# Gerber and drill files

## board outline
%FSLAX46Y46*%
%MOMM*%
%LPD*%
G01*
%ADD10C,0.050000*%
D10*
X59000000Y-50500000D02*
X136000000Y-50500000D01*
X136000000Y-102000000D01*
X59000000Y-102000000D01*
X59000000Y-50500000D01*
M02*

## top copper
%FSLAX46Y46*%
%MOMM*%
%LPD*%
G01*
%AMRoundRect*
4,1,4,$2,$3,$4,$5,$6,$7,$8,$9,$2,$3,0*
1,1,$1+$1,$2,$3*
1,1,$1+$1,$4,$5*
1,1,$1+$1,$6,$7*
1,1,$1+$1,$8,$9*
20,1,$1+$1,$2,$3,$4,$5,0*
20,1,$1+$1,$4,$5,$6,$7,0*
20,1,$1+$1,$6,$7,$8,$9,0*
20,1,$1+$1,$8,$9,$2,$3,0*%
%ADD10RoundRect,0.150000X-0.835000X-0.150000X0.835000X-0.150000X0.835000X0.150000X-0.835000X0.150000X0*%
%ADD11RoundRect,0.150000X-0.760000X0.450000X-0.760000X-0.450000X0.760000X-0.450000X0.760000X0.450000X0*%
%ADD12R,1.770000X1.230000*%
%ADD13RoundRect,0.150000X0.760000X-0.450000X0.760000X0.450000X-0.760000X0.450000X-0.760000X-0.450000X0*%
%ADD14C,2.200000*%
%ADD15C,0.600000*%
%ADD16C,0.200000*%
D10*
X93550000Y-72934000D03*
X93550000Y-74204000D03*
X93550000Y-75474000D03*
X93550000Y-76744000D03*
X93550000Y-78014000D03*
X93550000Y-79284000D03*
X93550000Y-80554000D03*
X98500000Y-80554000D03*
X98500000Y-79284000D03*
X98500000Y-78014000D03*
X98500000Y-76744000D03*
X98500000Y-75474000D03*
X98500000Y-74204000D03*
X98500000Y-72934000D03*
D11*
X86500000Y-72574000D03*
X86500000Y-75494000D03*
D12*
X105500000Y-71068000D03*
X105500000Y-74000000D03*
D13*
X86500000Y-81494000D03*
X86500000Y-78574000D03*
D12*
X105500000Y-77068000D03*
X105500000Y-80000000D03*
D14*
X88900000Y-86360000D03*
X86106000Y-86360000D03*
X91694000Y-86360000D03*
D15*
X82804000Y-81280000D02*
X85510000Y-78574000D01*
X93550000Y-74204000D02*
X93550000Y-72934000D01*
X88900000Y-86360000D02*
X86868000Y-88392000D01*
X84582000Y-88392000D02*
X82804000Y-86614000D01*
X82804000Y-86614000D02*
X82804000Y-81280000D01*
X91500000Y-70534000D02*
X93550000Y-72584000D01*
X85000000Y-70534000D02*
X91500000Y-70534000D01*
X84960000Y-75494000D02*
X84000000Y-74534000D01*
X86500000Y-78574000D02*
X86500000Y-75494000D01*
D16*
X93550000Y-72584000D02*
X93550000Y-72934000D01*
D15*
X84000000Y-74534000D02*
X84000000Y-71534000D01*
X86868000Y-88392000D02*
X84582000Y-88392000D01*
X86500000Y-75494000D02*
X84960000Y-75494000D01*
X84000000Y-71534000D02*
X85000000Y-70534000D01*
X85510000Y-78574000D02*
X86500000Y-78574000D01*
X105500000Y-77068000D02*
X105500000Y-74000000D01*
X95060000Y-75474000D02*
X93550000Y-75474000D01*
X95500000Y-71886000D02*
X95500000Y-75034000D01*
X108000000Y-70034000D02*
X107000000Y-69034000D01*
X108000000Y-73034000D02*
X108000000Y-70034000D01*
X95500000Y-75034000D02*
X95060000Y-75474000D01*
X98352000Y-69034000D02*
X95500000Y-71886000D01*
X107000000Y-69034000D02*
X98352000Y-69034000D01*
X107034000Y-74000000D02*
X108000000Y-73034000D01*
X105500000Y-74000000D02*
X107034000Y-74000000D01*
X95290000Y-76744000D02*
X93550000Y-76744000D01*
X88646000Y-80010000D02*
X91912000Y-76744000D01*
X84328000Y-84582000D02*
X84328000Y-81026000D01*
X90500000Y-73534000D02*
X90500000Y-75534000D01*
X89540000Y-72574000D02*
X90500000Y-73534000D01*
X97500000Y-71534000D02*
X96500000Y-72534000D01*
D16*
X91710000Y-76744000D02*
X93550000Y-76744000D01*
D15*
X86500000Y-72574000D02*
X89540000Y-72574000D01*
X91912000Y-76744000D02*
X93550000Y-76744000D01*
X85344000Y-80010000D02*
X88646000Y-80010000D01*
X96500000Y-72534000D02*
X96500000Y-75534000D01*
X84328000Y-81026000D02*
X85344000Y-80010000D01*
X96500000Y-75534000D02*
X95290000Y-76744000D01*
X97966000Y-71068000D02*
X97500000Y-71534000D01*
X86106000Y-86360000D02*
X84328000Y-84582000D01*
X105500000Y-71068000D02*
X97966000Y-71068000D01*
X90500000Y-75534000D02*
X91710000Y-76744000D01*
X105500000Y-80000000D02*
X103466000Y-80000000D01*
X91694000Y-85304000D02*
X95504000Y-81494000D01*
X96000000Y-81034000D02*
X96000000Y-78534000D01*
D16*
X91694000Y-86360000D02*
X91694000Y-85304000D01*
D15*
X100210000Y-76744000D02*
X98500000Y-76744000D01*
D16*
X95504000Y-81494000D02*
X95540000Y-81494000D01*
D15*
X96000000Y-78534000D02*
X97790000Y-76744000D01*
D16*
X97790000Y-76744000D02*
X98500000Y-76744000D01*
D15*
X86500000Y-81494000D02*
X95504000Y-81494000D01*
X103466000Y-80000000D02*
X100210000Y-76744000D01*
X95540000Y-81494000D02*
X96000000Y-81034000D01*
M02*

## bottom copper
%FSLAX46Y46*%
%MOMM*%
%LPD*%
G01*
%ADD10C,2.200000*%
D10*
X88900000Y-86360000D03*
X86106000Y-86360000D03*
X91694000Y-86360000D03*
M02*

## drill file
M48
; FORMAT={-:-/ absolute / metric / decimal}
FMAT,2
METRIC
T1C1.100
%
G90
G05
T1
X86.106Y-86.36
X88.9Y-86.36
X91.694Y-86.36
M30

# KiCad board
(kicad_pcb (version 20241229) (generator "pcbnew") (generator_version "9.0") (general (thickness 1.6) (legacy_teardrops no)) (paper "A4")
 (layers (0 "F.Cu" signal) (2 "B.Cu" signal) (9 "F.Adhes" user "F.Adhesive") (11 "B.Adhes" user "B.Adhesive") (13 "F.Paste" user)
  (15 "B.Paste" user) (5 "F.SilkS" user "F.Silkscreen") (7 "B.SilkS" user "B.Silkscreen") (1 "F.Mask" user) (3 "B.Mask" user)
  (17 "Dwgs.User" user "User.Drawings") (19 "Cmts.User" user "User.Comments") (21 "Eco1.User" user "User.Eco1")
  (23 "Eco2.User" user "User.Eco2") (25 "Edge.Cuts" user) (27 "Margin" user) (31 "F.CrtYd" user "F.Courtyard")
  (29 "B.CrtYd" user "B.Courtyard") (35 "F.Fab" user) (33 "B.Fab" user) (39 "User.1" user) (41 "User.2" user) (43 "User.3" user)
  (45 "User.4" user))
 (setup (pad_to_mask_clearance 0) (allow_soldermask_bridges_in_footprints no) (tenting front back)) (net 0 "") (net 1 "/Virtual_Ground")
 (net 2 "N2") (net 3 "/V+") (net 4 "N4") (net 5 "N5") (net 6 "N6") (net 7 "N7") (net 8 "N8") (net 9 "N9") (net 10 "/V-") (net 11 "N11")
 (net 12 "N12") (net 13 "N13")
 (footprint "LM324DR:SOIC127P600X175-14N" (layer "F.Cu") (at 96.025 76.744)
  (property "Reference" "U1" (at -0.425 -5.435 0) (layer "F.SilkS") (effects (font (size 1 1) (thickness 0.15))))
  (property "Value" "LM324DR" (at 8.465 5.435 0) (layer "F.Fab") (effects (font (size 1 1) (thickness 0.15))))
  (pad "1" smd roundrect (at -2.475 -3.81) (size 1.97 0.6) (layers "F.Cu" "F.Mask" "F.Paste") (roundrect_rratio 0.25)
   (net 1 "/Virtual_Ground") (solder_mask_margin 0.102))
  (pad "2" smd roundrect (at -2.475 -2.54) (size 1.97 0.6) (layers "F.Cu" "F.Mask" "F.Paste") (roundrect_rratio 0.25)
   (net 1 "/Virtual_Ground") (solder_mask_margin 0.102))
  (pad "3" smd roundrect (at -2.475 -1.27) (size 1.97 0.6) (layers "F.Cu" "F.Mask" "F.Paste") (roundrect_rratio 0.25) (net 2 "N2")
   (solder_mask_margin 0.102))
  (pad "4" smd roundrect (at -2.475 0) (size 1.97 0.6) (layers "F.Cu" "F.Mask" "F.Paste") (roundrect_rratio 0.25) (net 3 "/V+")
   (solder_mask_margin 0.102))
  (pad "5" smd roundrect (at -2.475 1.27) (size 1.97 0.6) (layers "F.Cu" "F.Mask" "F.Paste") (roundrect_rratio 0.25) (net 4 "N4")
   (solder_mask_margin 0.102))
  (pad "6" smd roundrect (at -2.475 2.54) (size 1.97 0.6) (layers "F.Cu" "F.Mask" "F.Paste") (roundrect_rratio 0.25) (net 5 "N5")
   (solder_mask_margin 0.102))
  (pad "7" smd roundrect (at -2.475 3.81) (size 1.97 0.6) (layers "F.Cu" "F.Mask" "F.Paste") (roundrect_rratio 0.25) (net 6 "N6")
   (solder_mask_margin 0.102))
  (pad "8" smd roundrect (at 2.475 3.81) (size 1.97 0.6) (layers "F.Cu" "F.Mask" "F.Paste") (roundrect_rratio 0.25) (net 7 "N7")
   (solder_mask_margin 0.102))
  (pad "9" smd roundrect (at 2.475 2.54) (size 1.97 0.6) (layers "F.Cu" "F.Mask" "F.Paste") (roundrect_rratio 0.25) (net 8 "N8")
   (solder_mask_margin 0.102))
  (pad "10" smd roundrect (at 2.475 1.27) (size 1.97 0.6) (layers "F.Cu" "F.Mask" "F.Paste") (roundrect_rratio 0.25) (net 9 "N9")
   (solder_mask_margin 0.102))
  (pad "11" smd roundrect (at 2.475 0) (size 1.97 0.6) (layers "F.Cu" "F.Mask" "F.Paste") (roundrect_rratio 0.25) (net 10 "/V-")
   (solder_mask_margin 0.102))
  (pad "12" smd roundrect (at 2.475 -1.27) (size 1.97 0.6) (layers "F.Cu" "F.Mask" "F.Paste") (roundrect_rratio 0.25) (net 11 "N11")
   (solder_mask_margin 0.102))
  (pad "13" smd roundrect (at 2.475 -2.54) (size 1.97 0.6) (layers "F.Cu" "F.Mask" "F.Paste") (roundrect_rratio 0.25) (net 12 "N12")
   (solder_mask_margin 0.102))
  (pad "14" smd roundrect (at 2.475 -3.81) (size 1.97 0.6) (layers "F.Cu" "F.Mask" "F.Paste") (roundrect_rratio 0.25) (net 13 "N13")
   (solder_mask_margin 0.102)))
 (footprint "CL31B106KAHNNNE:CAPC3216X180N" (layer "F.Cu") (at 86.5 74.034 -90)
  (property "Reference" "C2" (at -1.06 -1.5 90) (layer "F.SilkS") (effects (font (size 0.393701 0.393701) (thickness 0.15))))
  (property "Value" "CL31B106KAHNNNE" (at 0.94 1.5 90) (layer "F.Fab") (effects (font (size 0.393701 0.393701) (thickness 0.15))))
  (pad "1" smd roundrect (at -1.46 0 270) (size 1.2 1.82) (layers "F.Cu" "F.Mask" "F.Paste") (roundrect_rratio 0.125) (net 3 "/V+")
   (solder_mask_margin 0.102))
  (pad "2" smd roundrect (at 1.46 0 270) (size 1.2 1.82) (layers "F.Cu" "F.Mask" "F.Paste") (roundrect_rratio 0.125)
   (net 1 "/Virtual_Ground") (solder_mask_margin 0.102)))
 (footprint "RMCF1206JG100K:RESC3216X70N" (layer "F.Cu") (at 105.5 72.534 -90)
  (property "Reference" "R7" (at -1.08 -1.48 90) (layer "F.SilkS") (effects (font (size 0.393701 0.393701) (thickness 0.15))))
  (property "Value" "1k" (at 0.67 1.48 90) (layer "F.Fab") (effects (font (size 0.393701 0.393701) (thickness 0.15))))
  (pad "1" smd rect (at -1.466 0 270) (size 1.23 1.77) (layers "F.Cu" "F.Mask" "F.Paste") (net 3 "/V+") (solder_mask_margin 0.102))
  (pad "2" smd rect (at 1.466 0 270) (size 1.23 1.77) (layers "F.Cu" "F.Mask" "F.Paste") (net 2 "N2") (solder_mask_margin 0.102)))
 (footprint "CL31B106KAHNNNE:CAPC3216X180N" (layer "F.Cu") (at 86.5 80.034 90)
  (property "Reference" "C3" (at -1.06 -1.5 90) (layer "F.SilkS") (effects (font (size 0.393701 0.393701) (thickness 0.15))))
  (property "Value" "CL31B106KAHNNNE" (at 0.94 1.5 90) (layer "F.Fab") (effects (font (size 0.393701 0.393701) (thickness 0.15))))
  (pad "1" smd roundrect (at -1.46 0 90) (size 1.2 1.82) (layers "F.Cu" "F.Mask" "F.Paste") (roundrect_rratio 0.125) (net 10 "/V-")
   (solder_mask_margin 0.102))
  (pad "2" smd roundrect (at 1.46 0 90) (size 1.2 1.82) (layers "F.Cu" "F.Mask" "F.Paste") (roundrect_rratio 0.125)
   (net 1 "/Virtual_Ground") (solder_mask_margin 0.102)))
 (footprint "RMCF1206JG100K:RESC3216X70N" (layer "F.Cu") (at 105.5 78.534 -90)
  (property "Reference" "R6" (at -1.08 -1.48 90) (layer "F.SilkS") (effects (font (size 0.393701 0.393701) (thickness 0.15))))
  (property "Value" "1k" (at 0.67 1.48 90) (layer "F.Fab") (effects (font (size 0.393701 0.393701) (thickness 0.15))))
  (pad "1" smd rect (at -1.466 0 270) (size 1.23 1.77) (layers "F.Cu" "F.Mask" "F.Paste") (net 2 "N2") (solder_mask_margin 0.102))
  (pad "2" smd rect (at 1.466 0 270) (size 1.23 1.77) (layers "F.Cu" "F.Mask" "F.Paste") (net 10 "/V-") (solder_mask_margin 0.102)))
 (gr_rect (start 59 50.5) (end 136 102) (stroke (width 0.05) (type default)) (fill no) (layer "Edge.Cuts"))
 (segment (start 82.804 81.28) (end 85.51 78.574) (width 0.6) (layer "F.Cu") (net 1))
 (segment (start 93.55 74.204) (end 93.55 72.934) (width 0.6) (layer "F.Cu") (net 1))
 (segment (start 88.9 86.36) (end 86.868 88.392) (width 0.6) (layer "F.Cu") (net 1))
 (segment (start 84.582 88.392) (end 82.804 86.614) (width 0.6) (layer "F.Cu") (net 1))
 (segment (start 82.804 86.614) (end 82.804 81.28) (width 0.6) (layer "F.Cu") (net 1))
 (segment (start 91.5 70.534) (end 93.55 72.584) (width 0.6) (layer "F.Cu") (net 1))
 (segment (start 85 70.534) (end 91.5 70.534) (width 0.6) (layer "F.Cu") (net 1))
 (segment (start 84.96 75.494) (end 84 74.534) (width 0.6) (layer "F.Cu") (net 1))
 (segment (start 86.5 78.574) (end 86.5 75.494) (width 0.6) (layer "F.Cu") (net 1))
 (segment (start 93.55 72.584) (end 93.55 72.934) (width 0.2) (layer "F.Cu") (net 1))
 (segment (start 84 74.534) (end 84 71.534) (width 0.6) (layer "F.Cu") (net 1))
 (segment (start 86.868 88.392) (end 84.582 88.392) (width 0.6) (layer "F.Cu") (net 1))
 (segment (start 86.5 75.494) (end 84.96 75.494) (width 0.6) (layer "F.Cu") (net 1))
 (segment (start 84 71.534) (end 85 70.534) (width 0.6) (layer "F.Cu") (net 1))
 (segment (start 85.51 78.574) (end 86.5 78.574) (width 0.6) (layer "F.Cu") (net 1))
 (via (at 88.9 86.36) (size 2.2) (drill 1.1) (layers "F.Cu" "B.Cu") (free yes) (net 1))
 (segment (start 105.5 77.068) (end 105.5 74) (width 0.6) (layer "F.Cu") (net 2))
 (segment (start 95.06 75.474) (end 93.55 75.474) (width 0.6) (layer "F.Cu") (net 2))
 (segment (start 95.5 71.886) (end 95.5 75.034) (width 0.6) (layer "F.Cu") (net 2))
 (segment (start 108 70.034) (end 107 69.034) (width 0.6) (layer "F.Cu") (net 2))
 (segment (start 108 73.034) (end 108 70.034) (width 0.6) (layer "F.Cu") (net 2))
 (segment (start 95.5 75.034) (end 95.06 75.474) (width 0.6) (layer "F.Cu") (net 2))
 (segment (start 98.352 69.034) (end 95.5 71.886) (width 0.6) (layer "F.Cu") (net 2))
 (segment (start 107 69.034) (end 98.352 69.034) (width 0.6) (layer "F.Cu") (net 2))
 (segment (start 107.034 74) (end 108 73.034) (width 0.6) (layer "F.Cu") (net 2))
 (segment (start 105.5 74) (end 107.034 74) (width 0.6) (layer "F.Cu") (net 2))
 (segment (start 95.29 76.744) (end 93.55 76.744) (width 0.6) (layer "F.Cu") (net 3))
 (segment (start 88.646 80.01) (end 91.912 76.744) (width 0.6) (layer "F.Cu") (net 3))
 (segment (start 84.328 84.582) (end 84.328 81.026) (width 0.6) (layer "F.Cu") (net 3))
 (segment (start 90.5 73.534) (end 90.5 75.534) (width 0.6) (layer "F.Cu") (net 3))
 (segment (start 89.54 72.574) (end 90.5 73.534) (width 0.6) (layer "F.Cu") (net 3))
 (segment (start 97.5 71.534) (end 96.5 72.534) (width 0.6) (layer "F.Cu") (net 3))
 (segment (start 91.71 76.744) (end 93.55 76.744) (width 0.2) (layer "F.Cu") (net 3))
 (segment (start 86.5 72.574) (end 89.54 72.574) (width 0.6) (layer "F.Cu") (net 3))
 (segment (start 91.912 76.744) (end 93.55 76.744) (width 0.6) (layer "F.Cu") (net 3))
 (segment (start 85.344 80.01) (end 88.646 80.01) (width 0.6) (layer "F.Cu") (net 3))
 (segment (start 96.5 72.534) (end 96.5 75.534) (width 0.6) (layer "F.Cu") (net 3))
 (segment (start 84.328 81.026) (end 85.344 80.01) (width 0.6) (layer "F.Cu") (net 3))
 (segment (start 96.5 75.534) (end 95.29 76.744) (width 0.6) (layer "F.Cu") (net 3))
 (segment (start 97.966 71.068) (end 97.5 71.534) (width 0.6) (layer "F.Cu") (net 3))
 (segment (start 86.106 86.36) (end 84.328 84.582) (width 0.6) (layer "F.Cu") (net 3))
 (segment (start 105.5 71.068) (end 97.966 71.068) (width 0.6) (layer "F.Cu") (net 3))
 (segment (start 90.5 75.534) (end 91.71 76.744) (width 0.6) (layer "F.Cu") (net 3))
 (via (at 86.106 86.36) (size 2.2) (drill 1.1) (layers "F.Cu" "B.Cu") (free yes) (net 3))
 (segment (start 105.5 80) (end 103.466 80) (width 0.6) (layer "F.Cu") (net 10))
 (segment (start 91.694 85.304) (end 95.504 81.494) (width 0.6) (layer "F.Cu") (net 10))
 (segment (start 96 81.034) (end 96 78.534) (width 0.6) (layer "F.Cu") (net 10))
 (segment (start 91.694 86.36) (end 91.694 85.304) (width 0.2) (layer "F.Cu") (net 10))
 (segment (start 100.21 76.744) (end 98.5 76.744) (width 0.6) (layer "F.Cu") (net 10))
 (segment (start 95.504 81.494) (end 95.54 81.494) (width 0.2) (layer "F.Cu") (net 10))
 (segment (start 96 78.534) (end 97.79 76.744) (width 0.6) (layer "F.Cu") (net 10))
 (segment (start 97.79 76.744) (end 98.5 76.744) (width 0.2) (layer "F.Cu") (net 10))
 (segment (start 86.5 81.494) (end 95.504 81.494) (width 0.6) (layer "F.Cu") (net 10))
 (segment (start 103.466 80) (end 100.21 76.744) (width 0.6) (layer "F.Cu") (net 10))
 (segment (start 95.54 81.494) (end 96 81.034) (width 0.6) (layer "F.Cu") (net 10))
 (via (at 91.694 86.36) (size 2.2) (drill 1.1) (layers "F.Cu" "B.Cu") (free yes) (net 10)))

